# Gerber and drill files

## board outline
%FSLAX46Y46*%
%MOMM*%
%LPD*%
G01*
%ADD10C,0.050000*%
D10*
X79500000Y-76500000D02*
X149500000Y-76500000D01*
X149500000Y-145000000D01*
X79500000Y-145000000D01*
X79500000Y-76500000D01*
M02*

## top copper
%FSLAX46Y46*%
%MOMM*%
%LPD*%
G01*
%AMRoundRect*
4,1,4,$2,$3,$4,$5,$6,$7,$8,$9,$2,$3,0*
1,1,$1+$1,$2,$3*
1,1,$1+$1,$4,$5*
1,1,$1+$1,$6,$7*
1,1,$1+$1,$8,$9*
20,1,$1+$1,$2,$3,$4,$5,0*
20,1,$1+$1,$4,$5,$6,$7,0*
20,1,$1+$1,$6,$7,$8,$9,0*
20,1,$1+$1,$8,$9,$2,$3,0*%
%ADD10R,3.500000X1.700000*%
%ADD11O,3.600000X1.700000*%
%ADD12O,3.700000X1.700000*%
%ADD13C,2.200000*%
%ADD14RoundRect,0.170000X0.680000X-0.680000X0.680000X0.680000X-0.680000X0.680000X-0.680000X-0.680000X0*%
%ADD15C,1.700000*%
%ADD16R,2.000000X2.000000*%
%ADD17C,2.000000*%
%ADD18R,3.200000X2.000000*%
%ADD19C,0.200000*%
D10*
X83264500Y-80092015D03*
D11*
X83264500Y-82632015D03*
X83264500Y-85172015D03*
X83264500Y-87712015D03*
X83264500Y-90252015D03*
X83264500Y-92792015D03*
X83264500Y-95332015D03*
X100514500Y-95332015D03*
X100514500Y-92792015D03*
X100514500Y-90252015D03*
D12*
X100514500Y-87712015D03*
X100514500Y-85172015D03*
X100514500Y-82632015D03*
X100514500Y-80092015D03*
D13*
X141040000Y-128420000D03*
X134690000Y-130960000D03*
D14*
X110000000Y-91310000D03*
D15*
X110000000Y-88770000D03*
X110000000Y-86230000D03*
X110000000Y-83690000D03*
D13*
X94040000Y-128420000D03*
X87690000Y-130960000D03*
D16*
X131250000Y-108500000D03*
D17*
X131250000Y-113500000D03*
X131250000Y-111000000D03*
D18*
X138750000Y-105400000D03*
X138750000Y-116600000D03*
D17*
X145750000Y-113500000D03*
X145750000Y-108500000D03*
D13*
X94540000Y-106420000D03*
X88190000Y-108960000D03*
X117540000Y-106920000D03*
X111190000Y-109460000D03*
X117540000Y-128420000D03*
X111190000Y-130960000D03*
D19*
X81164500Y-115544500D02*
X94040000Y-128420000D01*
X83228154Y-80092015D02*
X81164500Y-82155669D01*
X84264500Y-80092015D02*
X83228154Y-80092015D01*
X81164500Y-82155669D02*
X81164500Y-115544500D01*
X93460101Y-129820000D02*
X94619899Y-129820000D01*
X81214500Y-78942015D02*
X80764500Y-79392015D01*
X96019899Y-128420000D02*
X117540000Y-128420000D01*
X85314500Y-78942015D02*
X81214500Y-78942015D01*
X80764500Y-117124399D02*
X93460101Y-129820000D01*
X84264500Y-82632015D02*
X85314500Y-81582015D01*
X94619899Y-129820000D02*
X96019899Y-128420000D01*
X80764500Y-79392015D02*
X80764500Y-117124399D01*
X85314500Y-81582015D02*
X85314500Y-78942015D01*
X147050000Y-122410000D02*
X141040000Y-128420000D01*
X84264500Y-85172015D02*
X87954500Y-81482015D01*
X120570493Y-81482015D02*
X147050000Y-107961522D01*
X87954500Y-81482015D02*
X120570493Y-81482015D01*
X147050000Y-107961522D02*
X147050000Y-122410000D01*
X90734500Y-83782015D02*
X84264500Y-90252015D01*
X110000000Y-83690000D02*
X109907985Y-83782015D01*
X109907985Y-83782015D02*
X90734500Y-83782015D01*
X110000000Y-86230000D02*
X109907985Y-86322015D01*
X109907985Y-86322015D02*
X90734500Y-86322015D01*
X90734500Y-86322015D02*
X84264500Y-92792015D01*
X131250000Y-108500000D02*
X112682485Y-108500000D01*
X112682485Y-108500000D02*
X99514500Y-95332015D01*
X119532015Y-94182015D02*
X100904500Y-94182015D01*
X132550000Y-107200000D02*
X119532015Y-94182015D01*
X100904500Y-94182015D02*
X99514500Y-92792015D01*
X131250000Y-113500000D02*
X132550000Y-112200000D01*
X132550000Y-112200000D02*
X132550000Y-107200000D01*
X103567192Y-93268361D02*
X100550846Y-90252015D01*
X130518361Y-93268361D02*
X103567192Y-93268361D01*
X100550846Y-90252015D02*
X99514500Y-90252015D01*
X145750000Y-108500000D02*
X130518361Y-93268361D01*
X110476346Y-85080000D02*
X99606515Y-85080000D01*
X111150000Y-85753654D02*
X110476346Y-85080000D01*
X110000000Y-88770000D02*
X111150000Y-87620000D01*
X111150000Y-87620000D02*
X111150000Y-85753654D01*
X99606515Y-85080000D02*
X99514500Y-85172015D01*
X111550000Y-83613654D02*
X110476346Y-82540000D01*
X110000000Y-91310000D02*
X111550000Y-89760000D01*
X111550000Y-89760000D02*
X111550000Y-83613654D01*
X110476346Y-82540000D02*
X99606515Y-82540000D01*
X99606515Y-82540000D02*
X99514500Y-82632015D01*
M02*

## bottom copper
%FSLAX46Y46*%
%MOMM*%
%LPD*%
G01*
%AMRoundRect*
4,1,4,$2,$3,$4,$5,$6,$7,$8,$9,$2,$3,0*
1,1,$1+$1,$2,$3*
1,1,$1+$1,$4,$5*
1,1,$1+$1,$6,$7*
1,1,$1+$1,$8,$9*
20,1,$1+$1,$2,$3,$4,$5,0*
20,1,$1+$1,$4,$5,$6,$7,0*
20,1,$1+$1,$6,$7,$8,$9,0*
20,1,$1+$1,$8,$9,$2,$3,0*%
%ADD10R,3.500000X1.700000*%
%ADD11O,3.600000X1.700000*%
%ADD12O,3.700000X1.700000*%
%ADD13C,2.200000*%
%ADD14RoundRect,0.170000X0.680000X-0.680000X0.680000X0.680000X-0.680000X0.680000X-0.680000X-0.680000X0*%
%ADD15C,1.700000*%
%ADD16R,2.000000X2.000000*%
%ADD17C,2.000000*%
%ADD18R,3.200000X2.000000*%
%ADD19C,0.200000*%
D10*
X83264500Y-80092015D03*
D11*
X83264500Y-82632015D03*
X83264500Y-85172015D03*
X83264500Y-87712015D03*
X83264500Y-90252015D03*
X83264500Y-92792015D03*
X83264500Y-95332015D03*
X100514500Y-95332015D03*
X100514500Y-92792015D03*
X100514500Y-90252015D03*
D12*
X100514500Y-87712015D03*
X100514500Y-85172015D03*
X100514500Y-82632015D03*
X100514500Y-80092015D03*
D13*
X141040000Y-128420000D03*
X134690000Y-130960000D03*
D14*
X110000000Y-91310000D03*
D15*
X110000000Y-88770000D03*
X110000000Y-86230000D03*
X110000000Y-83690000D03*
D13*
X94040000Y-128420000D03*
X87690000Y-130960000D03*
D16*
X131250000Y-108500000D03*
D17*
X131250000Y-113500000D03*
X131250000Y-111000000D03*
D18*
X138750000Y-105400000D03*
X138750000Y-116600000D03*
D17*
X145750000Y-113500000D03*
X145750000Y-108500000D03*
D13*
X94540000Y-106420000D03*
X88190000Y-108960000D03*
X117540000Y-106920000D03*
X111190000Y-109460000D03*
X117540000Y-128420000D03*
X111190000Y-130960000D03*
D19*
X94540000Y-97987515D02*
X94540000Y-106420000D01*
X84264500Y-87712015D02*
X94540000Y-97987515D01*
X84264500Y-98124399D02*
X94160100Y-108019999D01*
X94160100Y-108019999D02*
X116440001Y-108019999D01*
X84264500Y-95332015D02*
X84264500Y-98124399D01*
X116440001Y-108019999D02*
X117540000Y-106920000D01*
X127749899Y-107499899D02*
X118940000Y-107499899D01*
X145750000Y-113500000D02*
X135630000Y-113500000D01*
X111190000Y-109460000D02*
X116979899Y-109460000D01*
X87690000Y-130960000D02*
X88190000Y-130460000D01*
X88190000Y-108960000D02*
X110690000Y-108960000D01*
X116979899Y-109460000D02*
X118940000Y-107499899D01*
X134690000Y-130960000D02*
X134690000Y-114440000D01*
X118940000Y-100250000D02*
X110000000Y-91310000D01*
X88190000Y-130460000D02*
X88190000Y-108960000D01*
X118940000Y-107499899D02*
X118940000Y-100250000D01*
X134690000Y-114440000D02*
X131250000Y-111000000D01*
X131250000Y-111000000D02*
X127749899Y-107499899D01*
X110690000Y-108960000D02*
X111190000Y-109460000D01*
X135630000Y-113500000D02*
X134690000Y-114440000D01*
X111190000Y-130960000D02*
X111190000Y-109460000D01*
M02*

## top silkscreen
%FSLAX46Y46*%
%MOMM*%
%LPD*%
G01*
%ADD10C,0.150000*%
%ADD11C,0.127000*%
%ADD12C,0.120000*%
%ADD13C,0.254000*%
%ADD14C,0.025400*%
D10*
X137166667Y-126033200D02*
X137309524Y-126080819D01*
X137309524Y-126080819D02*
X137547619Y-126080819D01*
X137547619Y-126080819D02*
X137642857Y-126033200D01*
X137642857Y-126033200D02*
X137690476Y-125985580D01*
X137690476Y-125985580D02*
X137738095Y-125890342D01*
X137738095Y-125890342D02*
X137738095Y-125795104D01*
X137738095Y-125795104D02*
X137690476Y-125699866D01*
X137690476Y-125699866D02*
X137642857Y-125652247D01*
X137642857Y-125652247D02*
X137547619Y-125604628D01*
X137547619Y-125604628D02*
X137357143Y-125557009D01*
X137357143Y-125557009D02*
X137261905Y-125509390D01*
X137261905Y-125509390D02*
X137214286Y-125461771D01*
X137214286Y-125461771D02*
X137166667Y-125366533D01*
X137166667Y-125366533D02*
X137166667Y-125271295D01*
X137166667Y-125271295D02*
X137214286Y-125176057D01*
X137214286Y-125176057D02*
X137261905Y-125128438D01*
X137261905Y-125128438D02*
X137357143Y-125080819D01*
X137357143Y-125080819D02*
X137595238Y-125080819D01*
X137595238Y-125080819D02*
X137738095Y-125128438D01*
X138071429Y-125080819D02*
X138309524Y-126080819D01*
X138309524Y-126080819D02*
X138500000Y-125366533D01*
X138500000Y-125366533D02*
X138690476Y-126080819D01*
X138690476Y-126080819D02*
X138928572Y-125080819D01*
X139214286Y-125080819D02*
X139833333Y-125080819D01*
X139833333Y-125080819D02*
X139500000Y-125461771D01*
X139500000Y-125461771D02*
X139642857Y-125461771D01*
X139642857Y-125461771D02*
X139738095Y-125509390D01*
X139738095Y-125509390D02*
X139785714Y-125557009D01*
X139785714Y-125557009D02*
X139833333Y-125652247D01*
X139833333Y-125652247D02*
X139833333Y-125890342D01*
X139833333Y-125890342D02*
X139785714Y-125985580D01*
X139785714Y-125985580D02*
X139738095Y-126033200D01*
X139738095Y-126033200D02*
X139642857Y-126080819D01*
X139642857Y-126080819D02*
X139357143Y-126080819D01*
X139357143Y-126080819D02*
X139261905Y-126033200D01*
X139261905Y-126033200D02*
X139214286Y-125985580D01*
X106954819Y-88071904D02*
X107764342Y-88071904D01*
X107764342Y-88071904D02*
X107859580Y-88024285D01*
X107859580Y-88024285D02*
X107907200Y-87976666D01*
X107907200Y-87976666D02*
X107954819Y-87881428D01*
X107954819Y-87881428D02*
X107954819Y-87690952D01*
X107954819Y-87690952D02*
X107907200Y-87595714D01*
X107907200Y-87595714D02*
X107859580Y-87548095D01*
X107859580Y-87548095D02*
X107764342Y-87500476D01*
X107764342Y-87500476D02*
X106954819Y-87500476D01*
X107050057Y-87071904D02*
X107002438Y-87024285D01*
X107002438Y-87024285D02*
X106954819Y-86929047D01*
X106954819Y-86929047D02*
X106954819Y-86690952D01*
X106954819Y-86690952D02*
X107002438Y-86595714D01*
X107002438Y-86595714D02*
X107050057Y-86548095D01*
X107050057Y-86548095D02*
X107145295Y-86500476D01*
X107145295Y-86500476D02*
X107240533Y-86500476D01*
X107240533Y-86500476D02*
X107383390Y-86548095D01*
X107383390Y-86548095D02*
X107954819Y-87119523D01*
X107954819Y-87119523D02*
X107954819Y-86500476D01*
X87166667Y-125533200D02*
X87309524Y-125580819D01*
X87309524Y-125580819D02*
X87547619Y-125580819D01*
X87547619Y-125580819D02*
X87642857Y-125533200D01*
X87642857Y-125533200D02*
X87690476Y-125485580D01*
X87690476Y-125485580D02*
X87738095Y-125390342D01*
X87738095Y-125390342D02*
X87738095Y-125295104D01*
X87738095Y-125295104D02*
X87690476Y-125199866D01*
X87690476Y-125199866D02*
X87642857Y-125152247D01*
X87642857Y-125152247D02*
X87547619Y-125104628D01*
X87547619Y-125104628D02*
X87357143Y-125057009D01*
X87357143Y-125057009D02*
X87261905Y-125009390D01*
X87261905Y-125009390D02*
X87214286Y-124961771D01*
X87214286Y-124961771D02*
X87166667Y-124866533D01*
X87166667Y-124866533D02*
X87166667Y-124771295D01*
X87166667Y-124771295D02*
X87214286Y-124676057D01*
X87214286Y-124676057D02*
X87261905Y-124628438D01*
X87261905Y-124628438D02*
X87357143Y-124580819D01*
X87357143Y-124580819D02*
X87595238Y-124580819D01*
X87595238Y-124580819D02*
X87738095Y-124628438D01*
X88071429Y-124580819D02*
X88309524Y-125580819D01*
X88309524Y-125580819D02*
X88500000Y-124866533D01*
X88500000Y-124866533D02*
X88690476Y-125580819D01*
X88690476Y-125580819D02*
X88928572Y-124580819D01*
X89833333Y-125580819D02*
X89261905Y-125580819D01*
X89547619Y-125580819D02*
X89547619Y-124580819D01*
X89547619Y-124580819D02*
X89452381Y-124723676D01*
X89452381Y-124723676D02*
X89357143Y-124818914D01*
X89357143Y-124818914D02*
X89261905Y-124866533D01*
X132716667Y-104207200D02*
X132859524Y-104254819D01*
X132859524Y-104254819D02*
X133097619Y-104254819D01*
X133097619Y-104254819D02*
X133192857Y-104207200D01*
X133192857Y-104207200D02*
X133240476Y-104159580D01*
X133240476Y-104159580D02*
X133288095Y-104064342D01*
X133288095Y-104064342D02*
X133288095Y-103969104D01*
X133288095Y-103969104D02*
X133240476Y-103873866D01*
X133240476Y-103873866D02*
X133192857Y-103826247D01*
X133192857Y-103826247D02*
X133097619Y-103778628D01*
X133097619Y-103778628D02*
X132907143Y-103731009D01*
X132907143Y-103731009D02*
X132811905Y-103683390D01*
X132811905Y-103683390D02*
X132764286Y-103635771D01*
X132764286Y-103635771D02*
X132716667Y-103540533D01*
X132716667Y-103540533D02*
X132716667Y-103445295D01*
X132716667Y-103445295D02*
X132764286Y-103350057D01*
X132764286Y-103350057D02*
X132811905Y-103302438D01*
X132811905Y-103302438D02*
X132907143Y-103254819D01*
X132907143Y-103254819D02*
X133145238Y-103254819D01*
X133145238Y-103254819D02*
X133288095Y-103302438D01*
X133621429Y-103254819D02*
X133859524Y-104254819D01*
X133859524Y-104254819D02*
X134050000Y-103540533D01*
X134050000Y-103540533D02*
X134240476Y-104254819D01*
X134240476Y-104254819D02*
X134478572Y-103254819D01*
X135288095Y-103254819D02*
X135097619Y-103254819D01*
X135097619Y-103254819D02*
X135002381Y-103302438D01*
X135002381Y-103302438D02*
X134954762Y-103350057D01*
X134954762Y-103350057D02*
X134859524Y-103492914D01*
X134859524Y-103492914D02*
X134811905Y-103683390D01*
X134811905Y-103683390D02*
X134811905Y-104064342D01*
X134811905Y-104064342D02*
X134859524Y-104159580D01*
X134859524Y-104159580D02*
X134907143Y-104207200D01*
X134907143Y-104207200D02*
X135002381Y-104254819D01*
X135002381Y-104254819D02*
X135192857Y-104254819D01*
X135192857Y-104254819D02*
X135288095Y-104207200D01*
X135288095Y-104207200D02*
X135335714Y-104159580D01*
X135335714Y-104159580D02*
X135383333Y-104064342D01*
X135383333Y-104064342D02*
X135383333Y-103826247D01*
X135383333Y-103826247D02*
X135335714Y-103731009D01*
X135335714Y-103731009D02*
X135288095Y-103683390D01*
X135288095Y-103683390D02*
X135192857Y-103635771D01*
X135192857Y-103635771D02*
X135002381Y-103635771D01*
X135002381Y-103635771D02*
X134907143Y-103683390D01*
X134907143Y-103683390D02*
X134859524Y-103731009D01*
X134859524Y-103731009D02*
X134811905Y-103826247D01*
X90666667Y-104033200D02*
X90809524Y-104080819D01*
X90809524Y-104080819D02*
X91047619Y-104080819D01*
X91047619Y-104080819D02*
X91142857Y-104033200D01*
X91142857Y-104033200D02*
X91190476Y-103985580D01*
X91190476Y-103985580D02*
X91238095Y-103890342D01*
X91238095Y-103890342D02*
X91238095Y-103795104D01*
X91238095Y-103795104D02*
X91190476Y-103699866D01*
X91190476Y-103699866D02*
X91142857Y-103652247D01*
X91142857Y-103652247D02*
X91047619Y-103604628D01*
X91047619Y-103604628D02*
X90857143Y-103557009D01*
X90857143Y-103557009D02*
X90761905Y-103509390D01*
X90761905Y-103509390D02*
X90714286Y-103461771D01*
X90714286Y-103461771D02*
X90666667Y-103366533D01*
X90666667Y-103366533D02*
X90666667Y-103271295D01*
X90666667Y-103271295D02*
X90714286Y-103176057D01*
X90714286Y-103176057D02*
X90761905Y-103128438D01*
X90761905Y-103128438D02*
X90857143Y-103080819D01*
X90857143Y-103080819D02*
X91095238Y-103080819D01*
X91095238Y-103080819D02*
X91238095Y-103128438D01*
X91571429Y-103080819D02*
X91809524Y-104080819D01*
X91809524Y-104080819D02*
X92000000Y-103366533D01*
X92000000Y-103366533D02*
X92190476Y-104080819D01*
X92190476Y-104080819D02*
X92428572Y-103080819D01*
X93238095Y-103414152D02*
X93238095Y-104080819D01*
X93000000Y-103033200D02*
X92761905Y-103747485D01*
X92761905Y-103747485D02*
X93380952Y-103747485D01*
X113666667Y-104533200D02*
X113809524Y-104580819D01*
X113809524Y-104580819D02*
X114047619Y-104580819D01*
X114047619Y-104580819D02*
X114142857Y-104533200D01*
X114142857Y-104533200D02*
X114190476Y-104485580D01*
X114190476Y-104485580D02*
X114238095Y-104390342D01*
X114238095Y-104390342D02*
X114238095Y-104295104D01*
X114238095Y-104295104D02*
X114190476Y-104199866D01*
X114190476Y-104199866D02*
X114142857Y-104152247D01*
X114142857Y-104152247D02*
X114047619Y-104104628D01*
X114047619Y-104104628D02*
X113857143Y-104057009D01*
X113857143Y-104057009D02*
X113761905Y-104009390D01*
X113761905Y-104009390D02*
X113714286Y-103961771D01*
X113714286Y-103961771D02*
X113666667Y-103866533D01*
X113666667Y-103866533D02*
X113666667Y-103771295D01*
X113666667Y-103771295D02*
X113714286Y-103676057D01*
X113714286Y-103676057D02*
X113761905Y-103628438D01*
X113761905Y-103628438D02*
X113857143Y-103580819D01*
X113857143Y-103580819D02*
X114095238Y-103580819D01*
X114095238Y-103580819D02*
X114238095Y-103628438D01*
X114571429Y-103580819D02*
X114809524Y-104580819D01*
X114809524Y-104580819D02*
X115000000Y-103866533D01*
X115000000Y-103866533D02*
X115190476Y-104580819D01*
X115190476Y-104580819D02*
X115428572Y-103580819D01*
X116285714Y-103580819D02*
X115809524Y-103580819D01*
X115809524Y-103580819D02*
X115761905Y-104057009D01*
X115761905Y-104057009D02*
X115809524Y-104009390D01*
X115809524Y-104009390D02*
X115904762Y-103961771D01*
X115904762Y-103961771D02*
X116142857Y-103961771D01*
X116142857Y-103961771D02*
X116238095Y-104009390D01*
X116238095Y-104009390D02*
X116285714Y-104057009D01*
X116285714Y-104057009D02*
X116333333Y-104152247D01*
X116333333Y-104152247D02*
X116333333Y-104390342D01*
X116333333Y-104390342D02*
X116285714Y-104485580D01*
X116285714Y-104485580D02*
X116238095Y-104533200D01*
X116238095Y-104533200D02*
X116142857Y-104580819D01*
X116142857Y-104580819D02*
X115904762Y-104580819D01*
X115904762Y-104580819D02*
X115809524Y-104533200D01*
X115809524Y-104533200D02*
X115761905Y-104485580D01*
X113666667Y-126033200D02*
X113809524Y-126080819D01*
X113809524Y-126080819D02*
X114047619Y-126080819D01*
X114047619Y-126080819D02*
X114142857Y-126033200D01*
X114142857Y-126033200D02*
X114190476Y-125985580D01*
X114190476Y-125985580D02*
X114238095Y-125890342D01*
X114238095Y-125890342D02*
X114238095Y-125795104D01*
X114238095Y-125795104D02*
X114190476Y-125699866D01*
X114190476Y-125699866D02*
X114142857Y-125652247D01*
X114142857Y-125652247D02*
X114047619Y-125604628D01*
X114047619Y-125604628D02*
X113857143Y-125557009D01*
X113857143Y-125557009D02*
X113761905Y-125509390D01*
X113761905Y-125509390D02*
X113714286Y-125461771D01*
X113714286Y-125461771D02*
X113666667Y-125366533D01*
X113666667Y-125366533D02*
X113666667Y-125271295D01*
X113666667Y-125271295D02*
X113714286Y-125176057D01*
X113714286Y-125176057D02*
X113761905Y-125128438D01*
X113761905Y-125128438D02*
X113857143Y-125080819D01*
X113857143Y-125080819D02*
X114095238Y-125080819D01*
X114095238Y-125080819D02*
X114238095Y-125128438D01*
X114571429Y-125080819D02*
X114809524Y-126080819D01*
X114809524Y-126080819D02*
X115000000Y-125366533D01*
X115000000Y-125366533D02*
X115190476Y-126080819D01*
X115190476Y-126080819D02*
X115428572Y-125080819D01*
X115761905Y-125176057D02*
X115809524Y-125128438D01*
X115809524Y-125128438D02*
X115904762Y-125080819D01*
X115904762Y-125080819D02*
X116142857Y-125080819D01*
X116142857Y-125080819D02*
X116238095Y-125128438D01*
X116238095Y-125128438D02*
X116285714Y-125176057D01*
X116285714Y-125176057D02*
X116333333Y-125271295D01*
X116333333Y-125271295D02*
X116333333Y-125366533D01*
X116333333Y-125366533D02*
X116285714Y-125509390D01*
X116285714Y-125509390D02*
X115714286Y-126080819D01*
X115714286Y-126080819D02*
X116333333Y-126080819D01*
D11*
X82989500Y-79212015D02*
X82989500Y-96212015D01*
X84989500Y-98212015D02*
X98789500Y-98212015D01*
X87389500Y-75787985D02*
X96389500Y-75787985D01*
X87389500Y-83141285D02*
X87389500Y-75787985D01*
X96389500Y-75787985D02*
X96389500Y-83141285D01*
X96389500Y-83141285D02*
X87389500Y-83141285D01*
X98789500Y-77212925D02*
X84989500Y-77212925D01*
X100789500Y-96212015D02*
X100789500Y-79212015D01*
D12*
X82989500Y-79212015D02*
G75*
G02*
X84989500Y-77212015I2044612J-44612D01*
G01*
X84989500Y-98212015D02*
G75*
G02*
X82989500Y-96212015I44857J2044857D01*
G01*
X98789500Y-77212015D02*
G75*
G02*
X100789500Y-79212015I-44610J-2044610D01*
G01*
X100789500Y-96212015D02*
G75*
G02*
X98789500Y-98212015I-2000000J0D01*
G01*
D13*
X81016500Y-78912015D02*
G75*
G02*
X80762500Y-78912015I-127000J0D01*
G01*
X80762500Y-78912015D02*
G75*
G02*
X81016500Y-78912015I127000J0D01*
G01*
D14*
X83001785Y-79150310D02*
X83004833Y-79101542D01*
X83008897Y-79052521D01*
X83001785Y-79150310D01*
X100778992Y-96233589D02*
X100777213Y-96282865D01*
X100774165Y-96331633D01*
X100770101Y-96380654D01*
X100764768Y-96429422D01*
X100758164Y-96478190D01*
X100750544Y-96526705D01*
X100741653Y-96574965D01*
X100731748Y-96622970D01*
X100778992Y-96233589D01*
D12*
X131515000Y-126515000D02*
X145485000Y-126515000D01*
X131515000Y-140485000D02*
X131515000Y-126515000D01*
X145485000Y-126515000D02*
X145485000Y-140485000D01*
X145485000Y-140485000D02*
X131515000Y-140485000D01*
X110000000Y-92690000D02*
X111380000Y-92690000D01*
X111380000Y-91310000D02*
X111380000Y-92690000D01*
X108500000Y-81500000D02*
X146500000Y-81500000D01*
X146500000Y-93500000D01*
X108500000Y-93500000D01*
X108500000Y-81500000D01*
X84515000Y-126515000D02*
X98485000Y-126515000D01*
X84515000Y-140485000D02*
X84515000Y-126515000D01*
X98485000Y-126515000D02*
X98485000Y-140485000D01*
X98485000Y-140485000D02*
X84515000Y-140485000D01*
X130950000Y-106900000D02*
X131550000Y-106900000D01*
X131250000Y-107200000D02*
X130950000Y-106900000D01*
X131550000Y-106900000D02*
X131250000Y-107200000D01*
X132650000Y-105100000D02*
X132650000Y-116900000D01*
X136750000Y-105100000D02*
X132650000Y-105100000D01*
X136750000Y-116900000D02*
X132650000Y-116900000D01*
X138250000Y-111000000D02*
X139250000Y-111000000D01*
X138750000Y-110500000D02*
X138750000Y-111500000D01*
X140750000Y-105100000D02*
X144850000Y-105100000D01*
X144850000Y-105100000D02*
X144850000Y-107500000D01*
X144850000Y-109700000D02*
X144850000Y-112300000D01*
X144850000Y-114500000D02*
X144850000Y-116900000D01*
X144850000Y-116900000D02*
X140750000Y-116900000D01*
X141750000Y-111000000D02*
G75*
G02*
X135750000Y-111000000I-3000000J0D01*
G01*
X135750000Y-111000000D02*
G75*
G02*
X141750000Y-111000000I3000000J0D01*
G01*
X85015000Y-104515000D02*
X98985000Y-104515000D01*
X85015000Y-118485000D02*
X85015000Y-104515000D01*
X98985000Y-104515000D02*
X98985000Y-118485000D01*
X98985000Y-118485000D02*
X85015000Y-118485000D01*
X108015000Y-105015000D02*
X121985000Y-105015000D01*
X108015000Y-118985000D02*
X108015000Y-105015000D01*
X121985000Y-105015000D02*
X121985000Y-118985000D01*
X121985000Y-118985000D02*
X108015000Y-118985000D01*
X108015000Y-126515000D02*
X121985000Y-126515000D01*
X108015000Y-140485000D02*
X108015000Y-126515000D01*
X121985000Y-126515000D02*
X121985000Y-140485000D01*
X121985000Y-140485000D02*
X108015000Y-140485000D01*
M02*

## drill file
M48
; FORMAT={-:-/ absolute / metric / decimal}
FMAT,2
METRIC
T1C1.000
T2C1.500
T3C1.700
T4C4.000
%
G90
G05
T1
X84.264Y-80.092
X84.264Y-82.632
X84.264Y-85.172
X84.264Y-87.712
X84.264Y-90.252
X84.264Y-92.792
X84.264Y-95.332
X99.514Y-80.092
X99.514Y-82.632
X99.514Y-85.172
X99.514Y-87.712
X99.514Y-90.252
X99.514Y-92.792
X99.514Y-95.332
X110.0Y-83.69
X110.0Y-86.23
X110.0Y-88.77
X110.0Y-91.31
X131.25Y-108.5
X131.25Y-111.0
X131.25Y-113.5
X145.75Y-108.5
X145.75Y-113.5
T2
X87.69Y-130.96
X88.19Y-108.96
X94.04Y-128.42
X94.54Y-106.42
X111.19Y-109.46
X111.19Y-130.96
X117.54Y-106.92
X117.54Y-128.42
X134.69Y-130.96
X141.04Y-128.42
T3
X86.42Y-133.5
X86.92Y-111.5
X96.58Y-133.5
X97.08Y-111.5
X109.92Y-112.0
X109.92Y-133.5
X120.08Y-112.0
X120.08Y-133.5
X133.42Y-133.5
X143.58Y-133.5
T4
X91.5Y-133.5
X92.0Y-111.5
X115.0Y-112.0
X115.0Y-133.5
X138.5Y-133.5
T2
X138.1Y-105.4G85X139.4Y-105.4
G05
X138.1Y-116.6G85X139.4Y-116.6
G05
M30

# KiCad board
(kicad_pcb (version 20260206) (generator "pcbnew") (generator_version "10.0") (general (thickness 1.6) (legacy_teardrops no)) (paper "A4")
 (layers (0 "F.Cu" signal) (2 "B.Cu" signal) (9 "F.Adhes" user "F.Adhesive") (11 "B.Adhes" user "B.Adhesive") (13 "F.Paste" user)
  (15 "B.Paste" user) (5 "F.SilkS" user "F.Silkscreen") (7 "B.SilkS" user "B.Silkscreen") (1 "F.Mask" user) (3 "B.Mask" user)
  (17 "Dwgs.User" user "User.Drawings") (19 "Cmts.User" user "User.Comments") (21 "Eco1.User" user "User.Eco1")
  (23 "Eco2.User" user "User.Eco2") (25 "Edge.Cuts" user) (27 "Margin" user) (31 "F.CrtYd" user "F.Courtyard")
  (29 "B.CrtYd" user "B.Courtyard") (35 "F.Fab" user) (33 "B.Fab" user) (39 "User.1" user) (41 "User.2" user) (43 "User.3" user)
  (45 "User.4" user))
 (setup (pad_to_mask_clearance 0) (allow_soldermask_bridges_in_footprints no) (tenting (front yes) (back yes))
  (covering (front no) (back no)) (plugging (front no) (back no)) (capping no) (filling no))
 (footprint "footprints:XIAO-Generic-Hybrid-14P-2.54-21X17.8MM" (layer "F.Cu") (at 91.8895 87.712015)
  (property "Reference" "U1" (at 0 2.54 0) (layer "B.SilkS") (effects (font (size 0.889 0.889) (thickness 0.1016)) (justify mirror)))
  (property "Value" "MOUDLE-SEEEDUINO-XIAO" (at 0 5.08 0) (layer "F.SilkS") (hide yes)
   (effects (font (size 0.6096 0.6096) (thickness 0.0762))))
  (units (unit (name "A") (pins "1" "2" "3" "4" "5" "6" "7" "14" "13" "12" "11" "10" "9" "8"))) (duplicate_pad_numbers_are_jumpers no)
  (fp_line (start -8.9 -8.5) (end -8.9 8.5) (stroke (width 0.127) (type solid)) (layer "F.SilkS"))
  (fp_line (start -6.9 10.5) (end 6.9 10.5) (stroke (width 0.127) (type solid)) (layer "F.SilkS"))
  (fp_line (start -4.5 -11.92403) (end 4.5 -11.92403) (stroke (width 0.127) (type solid)) (layer "F.SilkS"))
  (fp_line (start -4.5 -4.57073) (end -4.5 -11.92403) (stroke (width 0.127) (type solid)) (layer "F.SilkS"))
  (fp_line (start 4.5 -11.92403) (end 4.5 -4.57073) (stroke (width 0.127) (type solid)) (layer "F.SilkS"))
  (fp_line (start 4.5 -4.57073) (end -4.5 -4.57073) (stroke (width 0.127) (type solid)) (layer "F.SilkS"))
  (fp_line (start 6.9 -10.49909) (end -6.9 -10.49909) (stroke (width 0.127) (type solid)) (layer "F.SilkS"))
  (fp_line (start 8.9 8.5) (end 8.9 -8.5) (stroke (width 0.127) (type solid)) (layer "F.SilkS"))
  (fp_arc (start -8.9 -8.5) (mid -8.301491 -9.901491) (end -6.9 -10.5) (stroke (width 0.12) (type solid)) (layer "F.SilkS"))
  (fp_arc (start -6.9 10.5) (mid -8.301423 9.901423) (end -8.9 8.5) (stroke (width 0.12) (type solid)) (layer "F.SilkS"))
  (fp_arc (start 6.9 -10.5) (mid 8.301491 -9.901491) (end 8.9 -8.5) (stroke (width 0.12) (type solid)) (layer "F.SilkS"))
  (fp_arc (start 8.9 8.5) (mid 8.314214 9.914214) (end 6.9 10.5) (stroke (width 0.12) (type solid)) (layer "F.SilkS"))
  (fp_circle (center -11 -8.8) (end -11 -9.054) (stroke (width 0) (type solid)) (fill yes) (layer "F.SilkS"))
  (fp_poly
   (pts (xy -8.887715 -8.561705) (xy -8.884667 -8.610473) (xy -8.880603 -8.659494)) (stroke (width 0.0254) (type solid)) (fill no)
   (layer "F.SilkS"))
  (fp_poly
   (pts (xy 8.889492 8.521574) (xy 8.887713 8.57085) (xy 8.884665 8.619618) (xy 8.880601 8.668639) (xy 8.875268 8.717407)
    (xy 8.868664 8.766175) (xy 8.861044 8.81469) (xy 8.852153 8.86295) (xy 8.842248 8.910955))
   (stroke (width 0.0254) (type solid)) (fill no) (layer "F.SilkS"))
  (pad "1" thru_hole rect (at -7.625 -7.62) (size 3.5 1.7) (drill 1 (offset -1 0)) (layers "*.Cu" "*.Mask") (remove_unused_layers no)
   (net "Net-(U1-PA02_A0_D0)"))
  (pad "2" thru_hole oval (at -7.625 -5.08) (size 3.6 1.7) (drill 1 (offset -1 0)) (layers "*.Cu" "*.Mask") (remove_unused_layers no)
   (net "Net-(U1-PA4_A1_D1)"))
  (pad "3" thru_hole oval (at -7.625 -2.54) (size 3.6 1.7) (drill 1 (offset -1 0)) (layers "*.Cu" "*.Mask") (remove_unused_layers no)
   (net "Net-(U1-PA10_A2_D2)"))
  (pad "4" thru_hole oval (at -7.625 0) (size 3.6 1.7) (drill 1 (offset -1 0)) (layers "*.Cu" "*.Mask") (remove_unused_layers no)
   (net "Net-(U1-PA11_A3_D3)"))
  (pad "5" thru_hole oval (at -7.625 2.54) (size 3.6 1.7) (drill 1 (offset -1 0)) (layers "*.Cu" "*.Mask") (remove_unused_layers no)
   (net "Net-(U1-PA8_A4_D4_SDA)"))
  (pad "6" thru_hole oval (at -7.625 5.08 180) (size 3.6 1.7) (drill 1 (offset 1 0)) (layers "*.Cu" "*.Mask") (remove_unused_layers no)
   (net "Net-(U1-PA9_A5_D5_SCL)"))
  (pad "7" thru_hole oval (at -7.625 7.62) (size 3.6 1.7) (drill 1 (offset -1 0)) (layers "*.Cu" "*.Mask") (remove_unused_layers no)
   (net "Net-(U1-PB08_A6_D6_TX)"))
  (pad "8" thru_hole oval (at 7.625 7.62) (size 3.6 1.7) (drill 1 (offset 1 0)) (layers "*.Cu" "*.Mask") (remove_unused_layers no)
   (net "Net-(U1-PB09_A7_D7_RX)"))
  (pad "9" thru_hole oval (at 7.625 5.08) (size 3.6 1.7) (drill 1 (offset 1 0)) (layers "*.Cu" "*.Mask") (remove_unused_layers no)
   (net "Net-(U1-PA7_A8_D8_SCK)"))
  (pad "10" thru_hole oval (at 7.625 2.54) (size 3.6 1.7) (drill 1 (offset 1 0)) (layers "*.Cu" "*.Mask") (remove_unused_layers no)
   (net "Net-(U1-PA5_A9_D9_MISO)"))
  (pad "11" thru_hole oval (at 7.625 0) (size 3.7 1.7) (drill 1 (offset 1 0)) (layers "*.Cu" "*.Mask") (remove_unused_layers no)
   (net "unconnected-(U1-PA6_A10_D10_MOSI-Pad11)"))
  (pad "12" thru_hole oval (at 7.625 -2.54) (size 3.7 1.7) (drill 1 (offset 1 0)) (layers "*.Cu" "*.Mask") (remove_unused_layers no)
   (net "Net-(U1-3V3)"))
  (pad "13" thru_hole oval (at 7.625 -5.08) (size 3.7 1.7) (drill 1 (offset 1 0)) (layers "*.Cu" "*.Mask") (remove_unused_layers no)
   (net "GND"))
  (pad "14" thru_hole oval (at 7.625 -7.62) (size 3.7 1.7) (drill 1 (offset 1 0)) (layers "*.Cu" "*.Mask") (remove_unused_layers no)
   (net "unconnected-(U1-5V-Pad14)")))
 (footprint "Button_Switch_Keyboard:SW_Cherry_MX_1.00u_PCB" (layer "F.Cu") (at 141.04 128.42)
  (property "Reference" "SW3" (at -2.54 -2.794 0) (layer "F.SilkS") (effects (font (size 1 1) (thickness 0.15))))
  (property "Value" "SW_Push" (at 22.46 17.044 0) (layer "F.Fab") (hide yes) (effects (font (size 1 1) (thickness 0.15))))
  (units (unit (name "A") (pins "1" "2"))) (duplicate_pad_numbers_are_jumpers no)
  (fp_line (start -9.525 -1.905) (end 4.445 -1.905) (stroke (width 0.12) (type solid)) (layer "F.SilkS"))
  (fp_line (start -9.525 12.065) (end -9.525 -1.905) (stroke (width 0.12) (type solid)) (layer "F.SilkS"))
  (fp_line (start 4.445 -1.905) (end 4.445 12.065) (stroke (width 0.12) (type solid)) (layer "F.SilkS"))
  (fp_line (start 4.445 12.065) (end -9.525 12.065) (stroke (width 0.12) (type solid)) (layer "F.SilkS"))
  (pad "" np_thru_hole circle (at -7.62 5.08) (size 1.7 1.7) (drill 1.7) (layers "*.Cu" "*.Mask"))
  (pad "" np_thru_hole circle (at -2.54 5.08) (size 4 4) (drill 4) (layers "*.Cu" "*.Mask"))
  (pad "" np_thru_hole circle (at 2.54 5.08) (size 1.7 1.7) (drill 1.7) (layers "*.Cu" "*.Mask"))
  (pad "1" thru_hole circle (at 0 0) (size 2.2 2.2) (drill 1.5) (layers "*.Cu" "*.Mask") (remove_unused_layers no)
   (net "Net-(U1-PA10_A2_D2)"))
  (pad "2" thru_hole circle (at -6.35 2.54) (size 2.2 2.2) (drill 1.5) (layers "*.Cu" "*.Mask") (remove_unused_layers no) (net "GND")))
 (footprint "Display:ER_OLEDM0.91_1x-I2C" (layer "F.Cu") (at 110 91.31 90)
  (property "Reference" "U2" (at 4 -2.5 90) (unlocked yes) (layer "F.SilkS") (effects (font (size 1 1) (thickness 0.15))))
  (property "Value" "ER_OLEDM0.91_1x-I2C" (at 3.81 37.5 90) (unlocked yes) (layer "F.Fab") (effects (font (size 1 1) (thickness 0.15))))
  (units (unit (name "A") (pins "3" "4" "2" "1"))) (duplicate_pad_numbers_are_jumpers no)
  (fp_line (start -1.38 0) (end -1.38 1.38) (stroke (width 0.12) (type solid)) (layer "F.SilkS"))
  (fp_line (start 0 1.38) (end -1.38 1.38) (stroke (width 0.12) (type solid)) (layer "F.SilkS"))
  (fp_rect (start -2.19 -1.5) (end 9.81 36.5) (stroke (width 0.12) (type solid)) (fill no) (layer "F.SilkS"))
  (pad "1" thru_hole roundrect (at 0 0 90) (size 1.7 1.7) (drill 1) (layers "*.Cu" "*.Mask") (remove_unused_layers no)
   (roundrect_rratio 0.1) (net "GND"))
  (pad "2" thru_hole circle (at 2.54 0 90) (size 1.7 1.7) (drill 1) (layers "*.Cu" "*.Mask") (remove_unused_layers no) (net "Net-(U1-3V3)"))
  (pad "3" thru_hole circle (at 5.08 0 90) (size 1.7 1.7) (drill 1) (layers "*.Cu" "*.Mask") (remove_unused_layers no)
   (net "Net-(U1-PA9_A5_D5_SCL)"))
  (pad "4" thru_hole circle (at 7.62 0 90) (size 1.7 1.7) (drill 1) (layers "*.Cu" "*.Mask") (remove_unused_layers no)
   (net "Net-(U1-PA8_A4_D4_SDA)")))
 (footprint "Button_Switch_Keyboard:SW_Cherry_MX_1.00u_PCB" (layer "F.Cu") (at 94.04 128.42)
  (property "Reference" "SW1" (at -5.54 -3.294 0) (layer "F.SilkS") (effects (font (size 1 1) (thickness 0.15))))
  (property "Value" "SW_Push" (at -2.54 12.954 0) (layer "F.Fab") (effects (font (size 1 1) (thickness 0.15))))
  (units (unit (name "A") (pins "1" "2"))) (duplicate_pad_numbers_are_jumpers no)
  (fp_line (start -9.525 -1.905) (end 4.445 -1.905) (stroke (width 0.12) (type solid)) (layer "F.SilkS"))
  (fp_line (start -9.525 12.065) (end -9.525 -1.905) (stroke (width 0.12) (type solid)) (layer "F.SilkS"))
  (fp_line (start 4.445 -1.905) (end 4.445 12.065) (stroke (width 0.12) (type solid)) (layer "F.SilkS"))
  (fp_line (start 4.445 12.065) (end -9.525 12.065) (stroke (width 0.12) (type solid)) (layer "F.SilkS"))
  (pad "" np_thru_hole circle (at -7.62 5.08) (size 1.7 1.7) (drill 1.7) (layers "*.Cu" "*.Mask"))
  (pad "" np_thru_hole circle (at -2.54 5.08) (size 4 4) (drill 4) (layers "*.Cu" "*.Mask"))
  (pad "" np_thru_hole circle (at 2.54 5.08) (size 1.7 1.7) (drill 1.7) (layers "*.Cu" "*.Mask"))
  (pad "1" thru_hole circle (at 0 0) (size 2.2 2.2) (drill 1.5) (layers "*.Cu" "*.Mask") (remove_unused_layers no)
   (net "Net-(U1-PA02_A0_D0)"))
  (pad "2" thru_hole circle (at -6.35 2.54) (size 2.2 2.2) (drill 1.5) (layers "*.Cu" "*.Mask") (remove_unused_layers no) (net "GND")))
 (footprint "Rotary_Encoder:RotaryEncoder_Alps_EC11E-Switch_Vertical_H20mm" (layer "F.Cu") (at 131.25 108.5)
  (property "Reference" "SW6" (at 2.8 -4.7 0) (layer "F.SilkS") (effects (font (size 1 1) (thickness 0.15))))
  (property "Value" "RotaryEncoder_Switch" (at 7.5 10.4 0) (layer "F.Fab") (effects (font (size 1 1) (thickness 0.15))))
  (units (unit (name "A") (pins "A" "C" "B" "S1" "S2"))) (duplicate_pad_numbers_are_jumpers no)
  (fp_line (start -0.3 -1.6) (end 0.3 -1.6) (stroke (width 0.12) (type solid)) (layer "F.SilkS"))
  (fp_line (start 0 -1.3) (end -0.3 -1.6) (stroke (width 0.12) (type solid)) (layer "F.SilkS"))
  (fp_line (start 0.3 -1.6) (end 0 -1.3) (stroke (width 0.12) (type solid)) (layer "F.SilkS"))
  (fp_line (start 1.4 -3.4) (end 1.4 8.4) (stroke (width 0.12) (type solid)) (layer "F.SilkS"))
  (fp_line (start 5.5 -3.4) (end 1.4 -3.4) (stroke (width 0.12) (type solid)) (layer "F.SilkS"))
  (fp_line (start 5.5 8.4) (end 1.4 8.4) (stroke (width 0.12) (type solid)) (layer "F.SilkS"))
  (fp_line (start 7 2.5) (end 8 2.5) (stroke (width 0.12) (type solid)) (layer "F.SilkS"))
  (fp_line (start 7.5 2) (end 7.5 3) (stroke (width 0.12) (type solid)) (layer "F.SilkS"))
  (fp_line (start 9.5 -3.4) (end 13.6 -3.4) (stroke (width 0.12) (type solid)) (layer "F.SilkS"))
  (fp_line (start 13.6 -3.4) (end 13.6 -1) (stroke (width 0.12) (type solid)) (layer "F.SilkS"))
  (fp_line (start 13.6 1.2) (end 13.6 3.8) (stroke (width 0.12) (type solid)) (layer "F.SilkS"))
  (fp_line (start 13.6 6) (end 13.6 8.4) (stroke (width 0.12) (type solid)) (layer "F.SilkS"))
  (fp_line (start 13.6 8.4) (end 9.5 8.4) (stroke (width 0.12) (type solid)) (layer "F.SilkS"))
  (fp_circle (center 7.5 2.5) (end 10.5 2.5) (stroke (width 0.12) (type solid)) (fill no) (layer "F.SilkS"))
  (pad "A" thru_hole rect (at 0 0) (size 2 2) (drill 1) (layers "*.Cu" "*.Mask") (remove_unused_layers no) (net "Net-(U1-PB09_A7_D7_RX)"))
  (pad "B" thru_hole circle (at 0 5) (size 2 2) (drill 1) (layers "*.Cu" "*.Mask") (remove_unused_layers no) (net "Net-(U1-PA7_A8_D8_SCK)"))
  (pad "C" thru_hole circle (at 0 2.5) (size 2 2) (drill 1) (layers "*.Cu" "*.Mask") (remove_unused_layers no) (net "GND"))
  (pad "MP" thru_hole rect (at 7.5 -3.1) (size 3.2 2) (drill oval 2.8 1.5) (layers "*.Cu" "*.Mask") (remove_unused_layers no))
  (pad "MP" thru_hole rect (at 7.5 8.1) (size 3.2 2) (drill oval 2.8 1.5) (layers "*.Cu" "*.Mask") (remove_unused_layers no))
  (pad "S1" thru_hole circle (at 14.5 5) (size 2 2) (drill 1) (layers "*.Cu" "*.Mask") (remove_unused_layers no) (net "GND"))
  (pad "S2" thru_hole circle (at 14.5 0) (size 2 2) (drill 1) (layers "*.Cu" "*.Mask") (remove_unused_layers no)
   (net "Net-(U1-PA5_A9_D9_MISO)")))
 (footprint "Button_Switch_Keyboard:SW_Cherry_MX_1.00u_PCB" (layer "F.Cu") (at 94.54 106.42)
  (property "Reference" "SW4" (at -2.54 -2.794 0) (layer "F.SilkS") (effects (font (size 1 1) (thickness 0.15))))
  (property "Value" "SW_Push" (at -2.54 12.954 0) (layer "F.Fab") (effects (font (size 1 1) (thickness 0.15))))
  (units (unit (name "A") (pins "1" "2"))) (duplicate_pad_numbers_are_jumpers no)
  (fp_line (start -9.525 -1.905) (end 4.445 -1.905) (stroke (width 0.12) (type solid)) (layer "F.SilkS"))
  (fp_line (start -9.525 12.065) (end -9.525 -1.905) (stroke (width 0.12) (type solid)) (layer "F.SilkS"))
  (fp_line (start 4.445 -1.905) (end 4.445 12.065) (stroke (width 0.12) (type solid)) (layer "F.SilkS"))
  (fp_line (start 4.445 12.065) (end -9.525 12.065) (stroke (width 0.12) (type solid)) (layer "F.SilkS"))
  (pad "" np_thru_hole circle (at -7.62 5.08) (size 1.7 1.7) (drill 1.7) (layers "*.Cu" "*.Mask"))
  (pad "" np_thru_hole circle (at -2.54 5.08) (size 4 4) (drill 4) (layers "*.Cu" "*.Mask"))
  (pad "" np_thru_hole circle (at 2.54 5.08) (size 1.7 1.7) (drill 1.7) (layers "*.Cu" "*.Mask"))
  (pad "1" thru_hole circle (at 0 0) (size 2.2 2.2) (drill 1.5) (layers "*.Cu" "*.Mask") (remove_unused_layers no)
   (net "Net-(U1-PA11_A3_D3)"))
  (pad "2" thru_hole circle (at -6.35 2.54) (size 2.2 2.2) (drill 1.5) (layers "*.Cu" "*.Mask") (remove_unused_layers no) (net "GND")))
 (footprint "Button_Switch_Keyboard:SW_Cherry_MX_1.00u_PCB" (layer "F.Cu") (at 117.54 106.92)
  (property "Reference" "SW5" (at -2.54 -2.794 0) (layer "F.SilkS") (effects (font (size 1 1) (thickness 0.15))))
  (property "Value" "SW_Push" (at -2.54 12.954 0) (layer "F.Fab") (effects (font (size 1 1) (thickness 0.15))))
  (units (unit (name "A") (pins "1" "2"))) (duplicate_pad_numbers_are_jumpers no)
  (fp_line (start -9.525 -1.905) (end 4.445 -1.905) (stroke (width 0.12) (type solid)) (layer "F.SilkS"))
  (fp_line (start -9.525 12.065) (end -9.525 -1.905) (stroke (width 0.12) (type solid)) (layer "F.SilkS"))
  (fp_line (start 4.445 -1.905) (end 4.445 12.065) (stroke (width 0.12) (type solid)) (layer "F.SilkS"))
  (fp_line (start 4.445 12.065) (end -9.525 12.065) (stroke (width 0.12) (type solid)) (layer "F.SilkS"))
  (pad "" np_thru_hole circle (at -7.62 5.08) (size 1.7 1.7) (drill 1.7) (layers "*.Cu" "*.Mask"))
  (pad "" np_thru_hole circle (at -2.54 5.08) (size 4 4) (drill 4) (layers "*.Cu" "*.Mask"))
  (pad "" np_thru_hole circle (at 2.54 5.08) (size 1.7 1.7) (drill 1.7) (layers "*.Cu" "*.Mask"))
  (pad "1" thru_hole circle (at 0 0) (size 2.2 2.2) (drill 1.5) (layers "*.Cu" "*.Mask") (remove_unused_layers no)
   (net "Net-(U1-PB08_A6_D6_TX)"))
  (pad "2" thru_hole circle (at -6.35 2.54) (size 2.2 2.2) (drill 1.5) (layers "*.Cu" "*.Mask") (remove_unused_layers no) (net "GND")))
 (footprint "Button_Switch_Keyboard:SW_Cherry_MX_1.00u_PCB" (layer "F.Cu") (at 117.54 128.42)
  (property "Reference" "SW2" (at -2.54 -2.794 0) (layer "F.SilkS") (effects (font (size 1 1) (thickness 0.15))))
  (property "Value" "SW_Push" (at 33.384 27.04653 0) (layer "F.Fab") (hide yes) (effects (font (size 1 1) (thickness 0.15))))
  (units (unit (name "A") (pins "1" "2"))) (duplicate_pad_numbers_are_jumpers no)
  (fp_line (start -9.525 -1.905) (end 4.445 -1.905) (stroke (width 0.12) (type solid)) (layer "F.SilkS"))
  (fp_line (start -9.525 12.065) (end -9.525 -1.905) (stroke (width 0.12) (type solid)) (layer "F.SilkS"))
  (fp_line (start 4.445 -1.905) (end 4.445 12.065) (stroke (width 0.12) (type solid)) (layer "F.SilkS"))
  (fp_line (start 4.445 12.065) (end -9.525 12.065) (stroke (width 0.12) (type solid)) (layer "F.SilkS"))
  (pad "" np_thru_hole circle (at -7.62 5.08) (size 1.7 1.7) (drill 1.7) (layers "*.Cu" "*.Mask"))
  (pad "" np_thru_hole circle (at -2.54 5.08) (size 4 4) (drill 4) (layers "*.Cu" "*.Mask"))
  (pad "" np_thru_hole circle (at 2.54 5.08) (size 1.7 1.7) (drill 1.7) (layers "*.Cu" "*.Mask"))
  (pad "1" thru_hole circle (at 0 0) (size 2.2 2.2) (drill 1.5) (layers "*.Cu" "*.Mask") (remove_unused_layers no)
   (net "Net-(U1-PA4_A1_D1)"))
  (pad "2" thru_hole circle (at -6.35 2.54) (size 2.2 2.2) (drill 1.5) (layers "*.Cu" "*.Mask") (remove_unused_layers no) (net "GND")))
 (gr_rect (start 79.5 76.5) (end 149.5 145) (stroke (width 0.05) (type default)) (fill no) (layer "Edge.Cuts"))
 (segment (start 81.1645 115.5445) (end 94.04 128.42) (width 0.2) (layer "F.Cu") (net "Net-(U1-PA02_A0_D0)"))
 (segment (start 83.228154 80.092015) (end 81.1645 82.155669) (width 0.2) (layer "F.Cu") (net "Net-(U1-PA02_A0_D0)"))
 (segment (start 84.2645 80.092015) (end 83.228154 80.092015) (width 0.2) (layer "F.Cu") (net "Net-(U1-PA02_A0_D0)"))
 (segment (start 81.1645 82.155669) (end 81.1645 115.5445) (width 0.2) (layer "F.Cu") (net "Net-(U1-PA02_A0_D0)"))
 (segment (start 93.460101 129.82) (end 94.619899 129.82) (width 0.2) (layer "F.Cu") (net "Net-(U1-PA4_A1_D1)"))
 (segment (start 81.2145 78.942015) (end 80.7645 79.392015) (width 0.2) (layer "F.Cu") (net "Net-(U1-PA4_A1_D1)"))
 (segment (start 96.019899 128.42) (end 117.54 128.42) (width 0.2) (layer "F.Cu") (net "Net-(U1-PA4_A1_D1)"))
 (segment (start 85.3145 78.942015) (end 81.2145 78.942015) (width 0.2) (layer "F.Cu") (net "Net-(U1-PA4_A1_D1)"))
 (segment (start 80.7645 117.124399) (end 93.460101 129.82) (width 0.2) (layer "F.Cu") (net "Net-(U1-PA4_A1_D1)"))
 (segment (start 84.2645 82.632015) (end 85.3145 81.582015) (width 0.2) (layer "F.Cu") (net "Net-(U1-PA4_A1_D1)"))
 (segment (start 94.619899 129.82) (end 96.019899 128.42) (width 0.2) (layer "F.Cu") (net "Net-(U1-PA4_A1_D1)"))
 (segment (start 80.7645 79.392015) (end 80.7645 117.124399) (width 0.2) (layer "F.Cu") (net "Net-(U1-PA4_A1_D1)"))
 (segment (start 85.3145 81.582015) (end 85.3145 78.942015) (width 0.2) (layer "F.Cu") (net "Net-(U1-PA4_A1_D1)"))
 (segment (start 147.05 122.41) (end 141.04 128.42) (width 0.2) (layer "F.Cu") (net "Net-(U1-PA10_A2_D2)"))
 (segment (start 84.2645 85.172015) (end 87.9545 81.482015) (width 0.2) (layer "F.Cu") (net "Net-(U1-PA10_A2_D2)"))
 (segment (start 120.570493 81.482015) (end 147.05 107.961522) (width 0.2) (layer "F.Cu") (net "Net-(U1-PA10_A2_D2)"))
 (segment (start 87.9545 81.482015) (end 120.570493 81.482015) (width 0.2) (layer "F.Cu") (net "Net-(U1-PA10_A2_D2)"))
 (segment (start 147.05 107.961522) (end 147.05 122.41) (width 0.2) (layer "F.Cu") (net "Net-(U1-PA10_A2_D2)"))
 (segment (start 94.54 97.987515) (end 94.54 106.42) (width 0.2) (layer "B.Cu") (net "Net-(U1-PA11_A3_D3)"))
 (segment (start 84.2645 87.712015) (end 94.54 97.987515) (width 0.2) (layer "B.Cu") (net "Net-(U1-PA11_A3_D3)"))
 (segment (start 90.7345 83.782015) (end 84.2645 90.252015) (width 0.2) (layer "F.Cu") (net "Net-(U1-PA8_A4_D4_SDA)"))
 (segment (start 110 83.69) (end 109.907985 83.782015) (width 0.2) (layer "F.Cu") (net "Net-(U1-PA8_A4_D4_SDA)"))
 (segment (start 109.907985 83.782015) (end 90.7345 83.782015) (width 0.2) (layer "F.Cu") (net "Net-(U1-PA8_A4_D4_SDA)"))
 (segment (start 110 86.23) (end 109.907985 86.322015) (width 0.2) (layer "F.Cu") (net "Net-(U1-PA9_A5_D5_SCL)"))
 (segment (start 109.907985 86.322015) (end 90.7345 86.322015) (width 0.2) (layer "F.Cu") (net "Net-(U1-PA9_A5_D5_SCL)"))
 (segment (start 90.7345 86.322015) (end 84.2645 92.792015) (width 0.2) (layer "F.Cu") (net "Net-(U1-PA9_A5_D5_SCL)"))
 (segment (start 84.2645 98.124399) (end 94.1601 108.019999) (width 0.2) (layer "B.Cu") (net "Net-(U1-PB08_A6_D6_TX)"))
 (segment (start 94.1601 108.019999) (end 116.440001 108.019999) (width 0.2) (layer "B.Cu") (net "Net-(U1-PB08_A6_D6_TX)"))
 (segment (start 84.2645 95.332015) (end 84.2645 98.124399) (width 0.2) (layer "B.Cu") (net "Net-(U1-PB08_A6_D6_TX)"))
 (segment (start 116.440001 108.019999) (end 117.54 106.92) (width 0.2) (layer "B.Cu") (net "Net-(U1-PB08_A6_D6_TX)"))
 (segment (start 131.25 108.5) (end 112.682485 108.5) (width 0.2) (layer "F.Cu") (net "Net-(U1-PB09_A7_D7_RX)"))
 (segment (start 112.682485 108.5) (end 99.5145 95.332015) (width 0.2) (layer "F.Cu") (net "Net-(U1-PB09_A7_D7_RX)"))
 (segment (start 119.532015 94.182015) (end 100.9045 94.182015) (width 0.2) (layer "F.Cu") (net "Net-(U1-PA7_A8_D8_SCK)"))
 (segment (start 132.55 107.2) (end 119.532015 94.182015) (width 0.2) (layer "F.Cu") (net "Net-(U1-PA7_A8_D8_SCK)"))
 (segment (start 100.9045 94.182015) (end 99.5145 92.792015) (width 0.2) (layer "F.Cu") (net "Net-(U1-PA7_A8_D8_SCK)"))
 (segment (start 131.25 113.5) (end 132.55 112.2) (width 0.2) (layer "F.Cu") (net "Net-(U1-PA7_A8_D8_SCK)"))
 (segment (start 132.55 112.2) (end 132.55 107.2) (width 0.2) (layer "F.Cu") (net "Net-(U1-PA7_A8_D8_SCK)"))
 (segment (start 103.567192 93.268361) (end 100.550846 90.252015) (width 0.2) (layer "F.Cu") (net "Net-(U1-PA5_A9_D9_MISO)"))
 (segment (start 130.518361 93.268361) (end 103.567192 93.268361) (width 0.2) (layer "F.Cu") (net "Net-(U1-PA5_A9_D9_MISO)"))
 (segment (start 100.550846 90.252015) (end 99.5145 90.252015) (width 0.2) (layer "F.Cu") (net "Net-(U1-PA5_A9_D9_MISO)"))
 (segment (start 145.75 108.5) (end 130.518361 93.268361) (width 0.2) (layer "F.Cu") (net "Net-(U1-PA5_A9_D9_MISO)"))
 (segment (start 110.476346 85.08) (end 99.606515 85.08) (width 0.2) (layer "F.Cu") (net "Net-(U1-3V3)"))
 (segment (start 111.15 85.753654) (end 110.476346 85.08) (width 0.2) (layer "F.Cu") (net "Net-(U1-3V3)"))
 (segment (start 110 88.77) (end 111.15 87.62) (width 0.2) (layer "F.Cu") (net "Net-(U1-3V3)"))
 (segment (start 111.15 87.62) (end 111.15 85.753654) (width 0.2) (layer "F.Cu") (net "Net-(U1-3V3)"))
 (segment (start 99.606515 85.08) (end 99.5145 85.172015) (width 0.2) (layer "F.Cu") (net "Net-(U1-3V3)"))
 (segment (start 111.55 83.613654) (end 110.476346 82.54) (width 0.2) (layer "F.Cu") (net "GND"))
 (segment (start 110 91.31) (end 111.55 89.76) (width 0.2) (layer "F.Cu") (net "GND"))
 (segment (start 111.55 89.76) (end 111.55 83.613654) (width 0.2) (layer "F.Cu") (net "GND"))
 (segment (start 110.476346 82.54) (end 99.606515 82.54) (width 0.2) (layer "F.Cu") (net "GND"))
 (segment (start 99.606515 82.54) (end 99.5145 82.632015) (width 0.2) (layer "F.Cu") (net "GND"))
 (segment (start 127.749899 107.499899) (end 118.94 107.499899) (width 0.2) (layer "B.Cu") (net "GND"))
 (segment (start 145.75 113.5) (end 135.63 113.5) (width 0.2) (layer "B.Cu") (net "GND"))
 (segment (start 111.19 109.46) (end 116.979899 109.46) (width 0.2) (layer "B.Cu") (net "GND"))
 (segment (start 87.69 130.96) (end 88.19 130.46) (width 0.2) (layer "B.Cu") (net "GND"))
 (segment (start 88.19 108.96) (end 110.69 108.96) (width 0.2) (layer "B.Cu") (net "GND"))
 (segment (start 116.979899 109.46) (end 118.94 107.499899) (width 0.2) (layer "B.Cu") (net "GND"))
 (segment (start 134.69 130.96) (end 134.69 114.44) (width 0.2) (layer "B.Cu") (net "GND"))
 (segment (start 118.94 100.25) (end 110 91.31) (width 0.2) (layer "B.Cu") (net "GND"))
 (segment (start 88.19 130.46) (end 88.19 108.96) (width 0.2) (layer "B.Cu") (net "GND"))
 (segment (start 118.94 107.499899) (end 118.94 100.25) (width 0.2) (layer "B.Cu") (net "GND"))
 (segment (start 134.69 114.44) (end 131.25 111) (width 0.2) (layer "B.Cu") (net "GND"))
 (segment (start 131.25 111) (end 127.749899 107.499899) (width 0.2) (layer "B.Cu") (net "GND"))
 (segment (start 110.69 108.96) (end 111.19 109.46) (width 0.2) (layer "B.Cu") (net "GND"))
 (segment (start 135.63 113.5) (end 134.69 114.44) (width 0.2) (layer "B.Cu") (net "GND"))
 (segment (start 111.19 130.96) (end 111.19 109.46) (width 0.2) (layer "B.Cu") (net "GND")))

